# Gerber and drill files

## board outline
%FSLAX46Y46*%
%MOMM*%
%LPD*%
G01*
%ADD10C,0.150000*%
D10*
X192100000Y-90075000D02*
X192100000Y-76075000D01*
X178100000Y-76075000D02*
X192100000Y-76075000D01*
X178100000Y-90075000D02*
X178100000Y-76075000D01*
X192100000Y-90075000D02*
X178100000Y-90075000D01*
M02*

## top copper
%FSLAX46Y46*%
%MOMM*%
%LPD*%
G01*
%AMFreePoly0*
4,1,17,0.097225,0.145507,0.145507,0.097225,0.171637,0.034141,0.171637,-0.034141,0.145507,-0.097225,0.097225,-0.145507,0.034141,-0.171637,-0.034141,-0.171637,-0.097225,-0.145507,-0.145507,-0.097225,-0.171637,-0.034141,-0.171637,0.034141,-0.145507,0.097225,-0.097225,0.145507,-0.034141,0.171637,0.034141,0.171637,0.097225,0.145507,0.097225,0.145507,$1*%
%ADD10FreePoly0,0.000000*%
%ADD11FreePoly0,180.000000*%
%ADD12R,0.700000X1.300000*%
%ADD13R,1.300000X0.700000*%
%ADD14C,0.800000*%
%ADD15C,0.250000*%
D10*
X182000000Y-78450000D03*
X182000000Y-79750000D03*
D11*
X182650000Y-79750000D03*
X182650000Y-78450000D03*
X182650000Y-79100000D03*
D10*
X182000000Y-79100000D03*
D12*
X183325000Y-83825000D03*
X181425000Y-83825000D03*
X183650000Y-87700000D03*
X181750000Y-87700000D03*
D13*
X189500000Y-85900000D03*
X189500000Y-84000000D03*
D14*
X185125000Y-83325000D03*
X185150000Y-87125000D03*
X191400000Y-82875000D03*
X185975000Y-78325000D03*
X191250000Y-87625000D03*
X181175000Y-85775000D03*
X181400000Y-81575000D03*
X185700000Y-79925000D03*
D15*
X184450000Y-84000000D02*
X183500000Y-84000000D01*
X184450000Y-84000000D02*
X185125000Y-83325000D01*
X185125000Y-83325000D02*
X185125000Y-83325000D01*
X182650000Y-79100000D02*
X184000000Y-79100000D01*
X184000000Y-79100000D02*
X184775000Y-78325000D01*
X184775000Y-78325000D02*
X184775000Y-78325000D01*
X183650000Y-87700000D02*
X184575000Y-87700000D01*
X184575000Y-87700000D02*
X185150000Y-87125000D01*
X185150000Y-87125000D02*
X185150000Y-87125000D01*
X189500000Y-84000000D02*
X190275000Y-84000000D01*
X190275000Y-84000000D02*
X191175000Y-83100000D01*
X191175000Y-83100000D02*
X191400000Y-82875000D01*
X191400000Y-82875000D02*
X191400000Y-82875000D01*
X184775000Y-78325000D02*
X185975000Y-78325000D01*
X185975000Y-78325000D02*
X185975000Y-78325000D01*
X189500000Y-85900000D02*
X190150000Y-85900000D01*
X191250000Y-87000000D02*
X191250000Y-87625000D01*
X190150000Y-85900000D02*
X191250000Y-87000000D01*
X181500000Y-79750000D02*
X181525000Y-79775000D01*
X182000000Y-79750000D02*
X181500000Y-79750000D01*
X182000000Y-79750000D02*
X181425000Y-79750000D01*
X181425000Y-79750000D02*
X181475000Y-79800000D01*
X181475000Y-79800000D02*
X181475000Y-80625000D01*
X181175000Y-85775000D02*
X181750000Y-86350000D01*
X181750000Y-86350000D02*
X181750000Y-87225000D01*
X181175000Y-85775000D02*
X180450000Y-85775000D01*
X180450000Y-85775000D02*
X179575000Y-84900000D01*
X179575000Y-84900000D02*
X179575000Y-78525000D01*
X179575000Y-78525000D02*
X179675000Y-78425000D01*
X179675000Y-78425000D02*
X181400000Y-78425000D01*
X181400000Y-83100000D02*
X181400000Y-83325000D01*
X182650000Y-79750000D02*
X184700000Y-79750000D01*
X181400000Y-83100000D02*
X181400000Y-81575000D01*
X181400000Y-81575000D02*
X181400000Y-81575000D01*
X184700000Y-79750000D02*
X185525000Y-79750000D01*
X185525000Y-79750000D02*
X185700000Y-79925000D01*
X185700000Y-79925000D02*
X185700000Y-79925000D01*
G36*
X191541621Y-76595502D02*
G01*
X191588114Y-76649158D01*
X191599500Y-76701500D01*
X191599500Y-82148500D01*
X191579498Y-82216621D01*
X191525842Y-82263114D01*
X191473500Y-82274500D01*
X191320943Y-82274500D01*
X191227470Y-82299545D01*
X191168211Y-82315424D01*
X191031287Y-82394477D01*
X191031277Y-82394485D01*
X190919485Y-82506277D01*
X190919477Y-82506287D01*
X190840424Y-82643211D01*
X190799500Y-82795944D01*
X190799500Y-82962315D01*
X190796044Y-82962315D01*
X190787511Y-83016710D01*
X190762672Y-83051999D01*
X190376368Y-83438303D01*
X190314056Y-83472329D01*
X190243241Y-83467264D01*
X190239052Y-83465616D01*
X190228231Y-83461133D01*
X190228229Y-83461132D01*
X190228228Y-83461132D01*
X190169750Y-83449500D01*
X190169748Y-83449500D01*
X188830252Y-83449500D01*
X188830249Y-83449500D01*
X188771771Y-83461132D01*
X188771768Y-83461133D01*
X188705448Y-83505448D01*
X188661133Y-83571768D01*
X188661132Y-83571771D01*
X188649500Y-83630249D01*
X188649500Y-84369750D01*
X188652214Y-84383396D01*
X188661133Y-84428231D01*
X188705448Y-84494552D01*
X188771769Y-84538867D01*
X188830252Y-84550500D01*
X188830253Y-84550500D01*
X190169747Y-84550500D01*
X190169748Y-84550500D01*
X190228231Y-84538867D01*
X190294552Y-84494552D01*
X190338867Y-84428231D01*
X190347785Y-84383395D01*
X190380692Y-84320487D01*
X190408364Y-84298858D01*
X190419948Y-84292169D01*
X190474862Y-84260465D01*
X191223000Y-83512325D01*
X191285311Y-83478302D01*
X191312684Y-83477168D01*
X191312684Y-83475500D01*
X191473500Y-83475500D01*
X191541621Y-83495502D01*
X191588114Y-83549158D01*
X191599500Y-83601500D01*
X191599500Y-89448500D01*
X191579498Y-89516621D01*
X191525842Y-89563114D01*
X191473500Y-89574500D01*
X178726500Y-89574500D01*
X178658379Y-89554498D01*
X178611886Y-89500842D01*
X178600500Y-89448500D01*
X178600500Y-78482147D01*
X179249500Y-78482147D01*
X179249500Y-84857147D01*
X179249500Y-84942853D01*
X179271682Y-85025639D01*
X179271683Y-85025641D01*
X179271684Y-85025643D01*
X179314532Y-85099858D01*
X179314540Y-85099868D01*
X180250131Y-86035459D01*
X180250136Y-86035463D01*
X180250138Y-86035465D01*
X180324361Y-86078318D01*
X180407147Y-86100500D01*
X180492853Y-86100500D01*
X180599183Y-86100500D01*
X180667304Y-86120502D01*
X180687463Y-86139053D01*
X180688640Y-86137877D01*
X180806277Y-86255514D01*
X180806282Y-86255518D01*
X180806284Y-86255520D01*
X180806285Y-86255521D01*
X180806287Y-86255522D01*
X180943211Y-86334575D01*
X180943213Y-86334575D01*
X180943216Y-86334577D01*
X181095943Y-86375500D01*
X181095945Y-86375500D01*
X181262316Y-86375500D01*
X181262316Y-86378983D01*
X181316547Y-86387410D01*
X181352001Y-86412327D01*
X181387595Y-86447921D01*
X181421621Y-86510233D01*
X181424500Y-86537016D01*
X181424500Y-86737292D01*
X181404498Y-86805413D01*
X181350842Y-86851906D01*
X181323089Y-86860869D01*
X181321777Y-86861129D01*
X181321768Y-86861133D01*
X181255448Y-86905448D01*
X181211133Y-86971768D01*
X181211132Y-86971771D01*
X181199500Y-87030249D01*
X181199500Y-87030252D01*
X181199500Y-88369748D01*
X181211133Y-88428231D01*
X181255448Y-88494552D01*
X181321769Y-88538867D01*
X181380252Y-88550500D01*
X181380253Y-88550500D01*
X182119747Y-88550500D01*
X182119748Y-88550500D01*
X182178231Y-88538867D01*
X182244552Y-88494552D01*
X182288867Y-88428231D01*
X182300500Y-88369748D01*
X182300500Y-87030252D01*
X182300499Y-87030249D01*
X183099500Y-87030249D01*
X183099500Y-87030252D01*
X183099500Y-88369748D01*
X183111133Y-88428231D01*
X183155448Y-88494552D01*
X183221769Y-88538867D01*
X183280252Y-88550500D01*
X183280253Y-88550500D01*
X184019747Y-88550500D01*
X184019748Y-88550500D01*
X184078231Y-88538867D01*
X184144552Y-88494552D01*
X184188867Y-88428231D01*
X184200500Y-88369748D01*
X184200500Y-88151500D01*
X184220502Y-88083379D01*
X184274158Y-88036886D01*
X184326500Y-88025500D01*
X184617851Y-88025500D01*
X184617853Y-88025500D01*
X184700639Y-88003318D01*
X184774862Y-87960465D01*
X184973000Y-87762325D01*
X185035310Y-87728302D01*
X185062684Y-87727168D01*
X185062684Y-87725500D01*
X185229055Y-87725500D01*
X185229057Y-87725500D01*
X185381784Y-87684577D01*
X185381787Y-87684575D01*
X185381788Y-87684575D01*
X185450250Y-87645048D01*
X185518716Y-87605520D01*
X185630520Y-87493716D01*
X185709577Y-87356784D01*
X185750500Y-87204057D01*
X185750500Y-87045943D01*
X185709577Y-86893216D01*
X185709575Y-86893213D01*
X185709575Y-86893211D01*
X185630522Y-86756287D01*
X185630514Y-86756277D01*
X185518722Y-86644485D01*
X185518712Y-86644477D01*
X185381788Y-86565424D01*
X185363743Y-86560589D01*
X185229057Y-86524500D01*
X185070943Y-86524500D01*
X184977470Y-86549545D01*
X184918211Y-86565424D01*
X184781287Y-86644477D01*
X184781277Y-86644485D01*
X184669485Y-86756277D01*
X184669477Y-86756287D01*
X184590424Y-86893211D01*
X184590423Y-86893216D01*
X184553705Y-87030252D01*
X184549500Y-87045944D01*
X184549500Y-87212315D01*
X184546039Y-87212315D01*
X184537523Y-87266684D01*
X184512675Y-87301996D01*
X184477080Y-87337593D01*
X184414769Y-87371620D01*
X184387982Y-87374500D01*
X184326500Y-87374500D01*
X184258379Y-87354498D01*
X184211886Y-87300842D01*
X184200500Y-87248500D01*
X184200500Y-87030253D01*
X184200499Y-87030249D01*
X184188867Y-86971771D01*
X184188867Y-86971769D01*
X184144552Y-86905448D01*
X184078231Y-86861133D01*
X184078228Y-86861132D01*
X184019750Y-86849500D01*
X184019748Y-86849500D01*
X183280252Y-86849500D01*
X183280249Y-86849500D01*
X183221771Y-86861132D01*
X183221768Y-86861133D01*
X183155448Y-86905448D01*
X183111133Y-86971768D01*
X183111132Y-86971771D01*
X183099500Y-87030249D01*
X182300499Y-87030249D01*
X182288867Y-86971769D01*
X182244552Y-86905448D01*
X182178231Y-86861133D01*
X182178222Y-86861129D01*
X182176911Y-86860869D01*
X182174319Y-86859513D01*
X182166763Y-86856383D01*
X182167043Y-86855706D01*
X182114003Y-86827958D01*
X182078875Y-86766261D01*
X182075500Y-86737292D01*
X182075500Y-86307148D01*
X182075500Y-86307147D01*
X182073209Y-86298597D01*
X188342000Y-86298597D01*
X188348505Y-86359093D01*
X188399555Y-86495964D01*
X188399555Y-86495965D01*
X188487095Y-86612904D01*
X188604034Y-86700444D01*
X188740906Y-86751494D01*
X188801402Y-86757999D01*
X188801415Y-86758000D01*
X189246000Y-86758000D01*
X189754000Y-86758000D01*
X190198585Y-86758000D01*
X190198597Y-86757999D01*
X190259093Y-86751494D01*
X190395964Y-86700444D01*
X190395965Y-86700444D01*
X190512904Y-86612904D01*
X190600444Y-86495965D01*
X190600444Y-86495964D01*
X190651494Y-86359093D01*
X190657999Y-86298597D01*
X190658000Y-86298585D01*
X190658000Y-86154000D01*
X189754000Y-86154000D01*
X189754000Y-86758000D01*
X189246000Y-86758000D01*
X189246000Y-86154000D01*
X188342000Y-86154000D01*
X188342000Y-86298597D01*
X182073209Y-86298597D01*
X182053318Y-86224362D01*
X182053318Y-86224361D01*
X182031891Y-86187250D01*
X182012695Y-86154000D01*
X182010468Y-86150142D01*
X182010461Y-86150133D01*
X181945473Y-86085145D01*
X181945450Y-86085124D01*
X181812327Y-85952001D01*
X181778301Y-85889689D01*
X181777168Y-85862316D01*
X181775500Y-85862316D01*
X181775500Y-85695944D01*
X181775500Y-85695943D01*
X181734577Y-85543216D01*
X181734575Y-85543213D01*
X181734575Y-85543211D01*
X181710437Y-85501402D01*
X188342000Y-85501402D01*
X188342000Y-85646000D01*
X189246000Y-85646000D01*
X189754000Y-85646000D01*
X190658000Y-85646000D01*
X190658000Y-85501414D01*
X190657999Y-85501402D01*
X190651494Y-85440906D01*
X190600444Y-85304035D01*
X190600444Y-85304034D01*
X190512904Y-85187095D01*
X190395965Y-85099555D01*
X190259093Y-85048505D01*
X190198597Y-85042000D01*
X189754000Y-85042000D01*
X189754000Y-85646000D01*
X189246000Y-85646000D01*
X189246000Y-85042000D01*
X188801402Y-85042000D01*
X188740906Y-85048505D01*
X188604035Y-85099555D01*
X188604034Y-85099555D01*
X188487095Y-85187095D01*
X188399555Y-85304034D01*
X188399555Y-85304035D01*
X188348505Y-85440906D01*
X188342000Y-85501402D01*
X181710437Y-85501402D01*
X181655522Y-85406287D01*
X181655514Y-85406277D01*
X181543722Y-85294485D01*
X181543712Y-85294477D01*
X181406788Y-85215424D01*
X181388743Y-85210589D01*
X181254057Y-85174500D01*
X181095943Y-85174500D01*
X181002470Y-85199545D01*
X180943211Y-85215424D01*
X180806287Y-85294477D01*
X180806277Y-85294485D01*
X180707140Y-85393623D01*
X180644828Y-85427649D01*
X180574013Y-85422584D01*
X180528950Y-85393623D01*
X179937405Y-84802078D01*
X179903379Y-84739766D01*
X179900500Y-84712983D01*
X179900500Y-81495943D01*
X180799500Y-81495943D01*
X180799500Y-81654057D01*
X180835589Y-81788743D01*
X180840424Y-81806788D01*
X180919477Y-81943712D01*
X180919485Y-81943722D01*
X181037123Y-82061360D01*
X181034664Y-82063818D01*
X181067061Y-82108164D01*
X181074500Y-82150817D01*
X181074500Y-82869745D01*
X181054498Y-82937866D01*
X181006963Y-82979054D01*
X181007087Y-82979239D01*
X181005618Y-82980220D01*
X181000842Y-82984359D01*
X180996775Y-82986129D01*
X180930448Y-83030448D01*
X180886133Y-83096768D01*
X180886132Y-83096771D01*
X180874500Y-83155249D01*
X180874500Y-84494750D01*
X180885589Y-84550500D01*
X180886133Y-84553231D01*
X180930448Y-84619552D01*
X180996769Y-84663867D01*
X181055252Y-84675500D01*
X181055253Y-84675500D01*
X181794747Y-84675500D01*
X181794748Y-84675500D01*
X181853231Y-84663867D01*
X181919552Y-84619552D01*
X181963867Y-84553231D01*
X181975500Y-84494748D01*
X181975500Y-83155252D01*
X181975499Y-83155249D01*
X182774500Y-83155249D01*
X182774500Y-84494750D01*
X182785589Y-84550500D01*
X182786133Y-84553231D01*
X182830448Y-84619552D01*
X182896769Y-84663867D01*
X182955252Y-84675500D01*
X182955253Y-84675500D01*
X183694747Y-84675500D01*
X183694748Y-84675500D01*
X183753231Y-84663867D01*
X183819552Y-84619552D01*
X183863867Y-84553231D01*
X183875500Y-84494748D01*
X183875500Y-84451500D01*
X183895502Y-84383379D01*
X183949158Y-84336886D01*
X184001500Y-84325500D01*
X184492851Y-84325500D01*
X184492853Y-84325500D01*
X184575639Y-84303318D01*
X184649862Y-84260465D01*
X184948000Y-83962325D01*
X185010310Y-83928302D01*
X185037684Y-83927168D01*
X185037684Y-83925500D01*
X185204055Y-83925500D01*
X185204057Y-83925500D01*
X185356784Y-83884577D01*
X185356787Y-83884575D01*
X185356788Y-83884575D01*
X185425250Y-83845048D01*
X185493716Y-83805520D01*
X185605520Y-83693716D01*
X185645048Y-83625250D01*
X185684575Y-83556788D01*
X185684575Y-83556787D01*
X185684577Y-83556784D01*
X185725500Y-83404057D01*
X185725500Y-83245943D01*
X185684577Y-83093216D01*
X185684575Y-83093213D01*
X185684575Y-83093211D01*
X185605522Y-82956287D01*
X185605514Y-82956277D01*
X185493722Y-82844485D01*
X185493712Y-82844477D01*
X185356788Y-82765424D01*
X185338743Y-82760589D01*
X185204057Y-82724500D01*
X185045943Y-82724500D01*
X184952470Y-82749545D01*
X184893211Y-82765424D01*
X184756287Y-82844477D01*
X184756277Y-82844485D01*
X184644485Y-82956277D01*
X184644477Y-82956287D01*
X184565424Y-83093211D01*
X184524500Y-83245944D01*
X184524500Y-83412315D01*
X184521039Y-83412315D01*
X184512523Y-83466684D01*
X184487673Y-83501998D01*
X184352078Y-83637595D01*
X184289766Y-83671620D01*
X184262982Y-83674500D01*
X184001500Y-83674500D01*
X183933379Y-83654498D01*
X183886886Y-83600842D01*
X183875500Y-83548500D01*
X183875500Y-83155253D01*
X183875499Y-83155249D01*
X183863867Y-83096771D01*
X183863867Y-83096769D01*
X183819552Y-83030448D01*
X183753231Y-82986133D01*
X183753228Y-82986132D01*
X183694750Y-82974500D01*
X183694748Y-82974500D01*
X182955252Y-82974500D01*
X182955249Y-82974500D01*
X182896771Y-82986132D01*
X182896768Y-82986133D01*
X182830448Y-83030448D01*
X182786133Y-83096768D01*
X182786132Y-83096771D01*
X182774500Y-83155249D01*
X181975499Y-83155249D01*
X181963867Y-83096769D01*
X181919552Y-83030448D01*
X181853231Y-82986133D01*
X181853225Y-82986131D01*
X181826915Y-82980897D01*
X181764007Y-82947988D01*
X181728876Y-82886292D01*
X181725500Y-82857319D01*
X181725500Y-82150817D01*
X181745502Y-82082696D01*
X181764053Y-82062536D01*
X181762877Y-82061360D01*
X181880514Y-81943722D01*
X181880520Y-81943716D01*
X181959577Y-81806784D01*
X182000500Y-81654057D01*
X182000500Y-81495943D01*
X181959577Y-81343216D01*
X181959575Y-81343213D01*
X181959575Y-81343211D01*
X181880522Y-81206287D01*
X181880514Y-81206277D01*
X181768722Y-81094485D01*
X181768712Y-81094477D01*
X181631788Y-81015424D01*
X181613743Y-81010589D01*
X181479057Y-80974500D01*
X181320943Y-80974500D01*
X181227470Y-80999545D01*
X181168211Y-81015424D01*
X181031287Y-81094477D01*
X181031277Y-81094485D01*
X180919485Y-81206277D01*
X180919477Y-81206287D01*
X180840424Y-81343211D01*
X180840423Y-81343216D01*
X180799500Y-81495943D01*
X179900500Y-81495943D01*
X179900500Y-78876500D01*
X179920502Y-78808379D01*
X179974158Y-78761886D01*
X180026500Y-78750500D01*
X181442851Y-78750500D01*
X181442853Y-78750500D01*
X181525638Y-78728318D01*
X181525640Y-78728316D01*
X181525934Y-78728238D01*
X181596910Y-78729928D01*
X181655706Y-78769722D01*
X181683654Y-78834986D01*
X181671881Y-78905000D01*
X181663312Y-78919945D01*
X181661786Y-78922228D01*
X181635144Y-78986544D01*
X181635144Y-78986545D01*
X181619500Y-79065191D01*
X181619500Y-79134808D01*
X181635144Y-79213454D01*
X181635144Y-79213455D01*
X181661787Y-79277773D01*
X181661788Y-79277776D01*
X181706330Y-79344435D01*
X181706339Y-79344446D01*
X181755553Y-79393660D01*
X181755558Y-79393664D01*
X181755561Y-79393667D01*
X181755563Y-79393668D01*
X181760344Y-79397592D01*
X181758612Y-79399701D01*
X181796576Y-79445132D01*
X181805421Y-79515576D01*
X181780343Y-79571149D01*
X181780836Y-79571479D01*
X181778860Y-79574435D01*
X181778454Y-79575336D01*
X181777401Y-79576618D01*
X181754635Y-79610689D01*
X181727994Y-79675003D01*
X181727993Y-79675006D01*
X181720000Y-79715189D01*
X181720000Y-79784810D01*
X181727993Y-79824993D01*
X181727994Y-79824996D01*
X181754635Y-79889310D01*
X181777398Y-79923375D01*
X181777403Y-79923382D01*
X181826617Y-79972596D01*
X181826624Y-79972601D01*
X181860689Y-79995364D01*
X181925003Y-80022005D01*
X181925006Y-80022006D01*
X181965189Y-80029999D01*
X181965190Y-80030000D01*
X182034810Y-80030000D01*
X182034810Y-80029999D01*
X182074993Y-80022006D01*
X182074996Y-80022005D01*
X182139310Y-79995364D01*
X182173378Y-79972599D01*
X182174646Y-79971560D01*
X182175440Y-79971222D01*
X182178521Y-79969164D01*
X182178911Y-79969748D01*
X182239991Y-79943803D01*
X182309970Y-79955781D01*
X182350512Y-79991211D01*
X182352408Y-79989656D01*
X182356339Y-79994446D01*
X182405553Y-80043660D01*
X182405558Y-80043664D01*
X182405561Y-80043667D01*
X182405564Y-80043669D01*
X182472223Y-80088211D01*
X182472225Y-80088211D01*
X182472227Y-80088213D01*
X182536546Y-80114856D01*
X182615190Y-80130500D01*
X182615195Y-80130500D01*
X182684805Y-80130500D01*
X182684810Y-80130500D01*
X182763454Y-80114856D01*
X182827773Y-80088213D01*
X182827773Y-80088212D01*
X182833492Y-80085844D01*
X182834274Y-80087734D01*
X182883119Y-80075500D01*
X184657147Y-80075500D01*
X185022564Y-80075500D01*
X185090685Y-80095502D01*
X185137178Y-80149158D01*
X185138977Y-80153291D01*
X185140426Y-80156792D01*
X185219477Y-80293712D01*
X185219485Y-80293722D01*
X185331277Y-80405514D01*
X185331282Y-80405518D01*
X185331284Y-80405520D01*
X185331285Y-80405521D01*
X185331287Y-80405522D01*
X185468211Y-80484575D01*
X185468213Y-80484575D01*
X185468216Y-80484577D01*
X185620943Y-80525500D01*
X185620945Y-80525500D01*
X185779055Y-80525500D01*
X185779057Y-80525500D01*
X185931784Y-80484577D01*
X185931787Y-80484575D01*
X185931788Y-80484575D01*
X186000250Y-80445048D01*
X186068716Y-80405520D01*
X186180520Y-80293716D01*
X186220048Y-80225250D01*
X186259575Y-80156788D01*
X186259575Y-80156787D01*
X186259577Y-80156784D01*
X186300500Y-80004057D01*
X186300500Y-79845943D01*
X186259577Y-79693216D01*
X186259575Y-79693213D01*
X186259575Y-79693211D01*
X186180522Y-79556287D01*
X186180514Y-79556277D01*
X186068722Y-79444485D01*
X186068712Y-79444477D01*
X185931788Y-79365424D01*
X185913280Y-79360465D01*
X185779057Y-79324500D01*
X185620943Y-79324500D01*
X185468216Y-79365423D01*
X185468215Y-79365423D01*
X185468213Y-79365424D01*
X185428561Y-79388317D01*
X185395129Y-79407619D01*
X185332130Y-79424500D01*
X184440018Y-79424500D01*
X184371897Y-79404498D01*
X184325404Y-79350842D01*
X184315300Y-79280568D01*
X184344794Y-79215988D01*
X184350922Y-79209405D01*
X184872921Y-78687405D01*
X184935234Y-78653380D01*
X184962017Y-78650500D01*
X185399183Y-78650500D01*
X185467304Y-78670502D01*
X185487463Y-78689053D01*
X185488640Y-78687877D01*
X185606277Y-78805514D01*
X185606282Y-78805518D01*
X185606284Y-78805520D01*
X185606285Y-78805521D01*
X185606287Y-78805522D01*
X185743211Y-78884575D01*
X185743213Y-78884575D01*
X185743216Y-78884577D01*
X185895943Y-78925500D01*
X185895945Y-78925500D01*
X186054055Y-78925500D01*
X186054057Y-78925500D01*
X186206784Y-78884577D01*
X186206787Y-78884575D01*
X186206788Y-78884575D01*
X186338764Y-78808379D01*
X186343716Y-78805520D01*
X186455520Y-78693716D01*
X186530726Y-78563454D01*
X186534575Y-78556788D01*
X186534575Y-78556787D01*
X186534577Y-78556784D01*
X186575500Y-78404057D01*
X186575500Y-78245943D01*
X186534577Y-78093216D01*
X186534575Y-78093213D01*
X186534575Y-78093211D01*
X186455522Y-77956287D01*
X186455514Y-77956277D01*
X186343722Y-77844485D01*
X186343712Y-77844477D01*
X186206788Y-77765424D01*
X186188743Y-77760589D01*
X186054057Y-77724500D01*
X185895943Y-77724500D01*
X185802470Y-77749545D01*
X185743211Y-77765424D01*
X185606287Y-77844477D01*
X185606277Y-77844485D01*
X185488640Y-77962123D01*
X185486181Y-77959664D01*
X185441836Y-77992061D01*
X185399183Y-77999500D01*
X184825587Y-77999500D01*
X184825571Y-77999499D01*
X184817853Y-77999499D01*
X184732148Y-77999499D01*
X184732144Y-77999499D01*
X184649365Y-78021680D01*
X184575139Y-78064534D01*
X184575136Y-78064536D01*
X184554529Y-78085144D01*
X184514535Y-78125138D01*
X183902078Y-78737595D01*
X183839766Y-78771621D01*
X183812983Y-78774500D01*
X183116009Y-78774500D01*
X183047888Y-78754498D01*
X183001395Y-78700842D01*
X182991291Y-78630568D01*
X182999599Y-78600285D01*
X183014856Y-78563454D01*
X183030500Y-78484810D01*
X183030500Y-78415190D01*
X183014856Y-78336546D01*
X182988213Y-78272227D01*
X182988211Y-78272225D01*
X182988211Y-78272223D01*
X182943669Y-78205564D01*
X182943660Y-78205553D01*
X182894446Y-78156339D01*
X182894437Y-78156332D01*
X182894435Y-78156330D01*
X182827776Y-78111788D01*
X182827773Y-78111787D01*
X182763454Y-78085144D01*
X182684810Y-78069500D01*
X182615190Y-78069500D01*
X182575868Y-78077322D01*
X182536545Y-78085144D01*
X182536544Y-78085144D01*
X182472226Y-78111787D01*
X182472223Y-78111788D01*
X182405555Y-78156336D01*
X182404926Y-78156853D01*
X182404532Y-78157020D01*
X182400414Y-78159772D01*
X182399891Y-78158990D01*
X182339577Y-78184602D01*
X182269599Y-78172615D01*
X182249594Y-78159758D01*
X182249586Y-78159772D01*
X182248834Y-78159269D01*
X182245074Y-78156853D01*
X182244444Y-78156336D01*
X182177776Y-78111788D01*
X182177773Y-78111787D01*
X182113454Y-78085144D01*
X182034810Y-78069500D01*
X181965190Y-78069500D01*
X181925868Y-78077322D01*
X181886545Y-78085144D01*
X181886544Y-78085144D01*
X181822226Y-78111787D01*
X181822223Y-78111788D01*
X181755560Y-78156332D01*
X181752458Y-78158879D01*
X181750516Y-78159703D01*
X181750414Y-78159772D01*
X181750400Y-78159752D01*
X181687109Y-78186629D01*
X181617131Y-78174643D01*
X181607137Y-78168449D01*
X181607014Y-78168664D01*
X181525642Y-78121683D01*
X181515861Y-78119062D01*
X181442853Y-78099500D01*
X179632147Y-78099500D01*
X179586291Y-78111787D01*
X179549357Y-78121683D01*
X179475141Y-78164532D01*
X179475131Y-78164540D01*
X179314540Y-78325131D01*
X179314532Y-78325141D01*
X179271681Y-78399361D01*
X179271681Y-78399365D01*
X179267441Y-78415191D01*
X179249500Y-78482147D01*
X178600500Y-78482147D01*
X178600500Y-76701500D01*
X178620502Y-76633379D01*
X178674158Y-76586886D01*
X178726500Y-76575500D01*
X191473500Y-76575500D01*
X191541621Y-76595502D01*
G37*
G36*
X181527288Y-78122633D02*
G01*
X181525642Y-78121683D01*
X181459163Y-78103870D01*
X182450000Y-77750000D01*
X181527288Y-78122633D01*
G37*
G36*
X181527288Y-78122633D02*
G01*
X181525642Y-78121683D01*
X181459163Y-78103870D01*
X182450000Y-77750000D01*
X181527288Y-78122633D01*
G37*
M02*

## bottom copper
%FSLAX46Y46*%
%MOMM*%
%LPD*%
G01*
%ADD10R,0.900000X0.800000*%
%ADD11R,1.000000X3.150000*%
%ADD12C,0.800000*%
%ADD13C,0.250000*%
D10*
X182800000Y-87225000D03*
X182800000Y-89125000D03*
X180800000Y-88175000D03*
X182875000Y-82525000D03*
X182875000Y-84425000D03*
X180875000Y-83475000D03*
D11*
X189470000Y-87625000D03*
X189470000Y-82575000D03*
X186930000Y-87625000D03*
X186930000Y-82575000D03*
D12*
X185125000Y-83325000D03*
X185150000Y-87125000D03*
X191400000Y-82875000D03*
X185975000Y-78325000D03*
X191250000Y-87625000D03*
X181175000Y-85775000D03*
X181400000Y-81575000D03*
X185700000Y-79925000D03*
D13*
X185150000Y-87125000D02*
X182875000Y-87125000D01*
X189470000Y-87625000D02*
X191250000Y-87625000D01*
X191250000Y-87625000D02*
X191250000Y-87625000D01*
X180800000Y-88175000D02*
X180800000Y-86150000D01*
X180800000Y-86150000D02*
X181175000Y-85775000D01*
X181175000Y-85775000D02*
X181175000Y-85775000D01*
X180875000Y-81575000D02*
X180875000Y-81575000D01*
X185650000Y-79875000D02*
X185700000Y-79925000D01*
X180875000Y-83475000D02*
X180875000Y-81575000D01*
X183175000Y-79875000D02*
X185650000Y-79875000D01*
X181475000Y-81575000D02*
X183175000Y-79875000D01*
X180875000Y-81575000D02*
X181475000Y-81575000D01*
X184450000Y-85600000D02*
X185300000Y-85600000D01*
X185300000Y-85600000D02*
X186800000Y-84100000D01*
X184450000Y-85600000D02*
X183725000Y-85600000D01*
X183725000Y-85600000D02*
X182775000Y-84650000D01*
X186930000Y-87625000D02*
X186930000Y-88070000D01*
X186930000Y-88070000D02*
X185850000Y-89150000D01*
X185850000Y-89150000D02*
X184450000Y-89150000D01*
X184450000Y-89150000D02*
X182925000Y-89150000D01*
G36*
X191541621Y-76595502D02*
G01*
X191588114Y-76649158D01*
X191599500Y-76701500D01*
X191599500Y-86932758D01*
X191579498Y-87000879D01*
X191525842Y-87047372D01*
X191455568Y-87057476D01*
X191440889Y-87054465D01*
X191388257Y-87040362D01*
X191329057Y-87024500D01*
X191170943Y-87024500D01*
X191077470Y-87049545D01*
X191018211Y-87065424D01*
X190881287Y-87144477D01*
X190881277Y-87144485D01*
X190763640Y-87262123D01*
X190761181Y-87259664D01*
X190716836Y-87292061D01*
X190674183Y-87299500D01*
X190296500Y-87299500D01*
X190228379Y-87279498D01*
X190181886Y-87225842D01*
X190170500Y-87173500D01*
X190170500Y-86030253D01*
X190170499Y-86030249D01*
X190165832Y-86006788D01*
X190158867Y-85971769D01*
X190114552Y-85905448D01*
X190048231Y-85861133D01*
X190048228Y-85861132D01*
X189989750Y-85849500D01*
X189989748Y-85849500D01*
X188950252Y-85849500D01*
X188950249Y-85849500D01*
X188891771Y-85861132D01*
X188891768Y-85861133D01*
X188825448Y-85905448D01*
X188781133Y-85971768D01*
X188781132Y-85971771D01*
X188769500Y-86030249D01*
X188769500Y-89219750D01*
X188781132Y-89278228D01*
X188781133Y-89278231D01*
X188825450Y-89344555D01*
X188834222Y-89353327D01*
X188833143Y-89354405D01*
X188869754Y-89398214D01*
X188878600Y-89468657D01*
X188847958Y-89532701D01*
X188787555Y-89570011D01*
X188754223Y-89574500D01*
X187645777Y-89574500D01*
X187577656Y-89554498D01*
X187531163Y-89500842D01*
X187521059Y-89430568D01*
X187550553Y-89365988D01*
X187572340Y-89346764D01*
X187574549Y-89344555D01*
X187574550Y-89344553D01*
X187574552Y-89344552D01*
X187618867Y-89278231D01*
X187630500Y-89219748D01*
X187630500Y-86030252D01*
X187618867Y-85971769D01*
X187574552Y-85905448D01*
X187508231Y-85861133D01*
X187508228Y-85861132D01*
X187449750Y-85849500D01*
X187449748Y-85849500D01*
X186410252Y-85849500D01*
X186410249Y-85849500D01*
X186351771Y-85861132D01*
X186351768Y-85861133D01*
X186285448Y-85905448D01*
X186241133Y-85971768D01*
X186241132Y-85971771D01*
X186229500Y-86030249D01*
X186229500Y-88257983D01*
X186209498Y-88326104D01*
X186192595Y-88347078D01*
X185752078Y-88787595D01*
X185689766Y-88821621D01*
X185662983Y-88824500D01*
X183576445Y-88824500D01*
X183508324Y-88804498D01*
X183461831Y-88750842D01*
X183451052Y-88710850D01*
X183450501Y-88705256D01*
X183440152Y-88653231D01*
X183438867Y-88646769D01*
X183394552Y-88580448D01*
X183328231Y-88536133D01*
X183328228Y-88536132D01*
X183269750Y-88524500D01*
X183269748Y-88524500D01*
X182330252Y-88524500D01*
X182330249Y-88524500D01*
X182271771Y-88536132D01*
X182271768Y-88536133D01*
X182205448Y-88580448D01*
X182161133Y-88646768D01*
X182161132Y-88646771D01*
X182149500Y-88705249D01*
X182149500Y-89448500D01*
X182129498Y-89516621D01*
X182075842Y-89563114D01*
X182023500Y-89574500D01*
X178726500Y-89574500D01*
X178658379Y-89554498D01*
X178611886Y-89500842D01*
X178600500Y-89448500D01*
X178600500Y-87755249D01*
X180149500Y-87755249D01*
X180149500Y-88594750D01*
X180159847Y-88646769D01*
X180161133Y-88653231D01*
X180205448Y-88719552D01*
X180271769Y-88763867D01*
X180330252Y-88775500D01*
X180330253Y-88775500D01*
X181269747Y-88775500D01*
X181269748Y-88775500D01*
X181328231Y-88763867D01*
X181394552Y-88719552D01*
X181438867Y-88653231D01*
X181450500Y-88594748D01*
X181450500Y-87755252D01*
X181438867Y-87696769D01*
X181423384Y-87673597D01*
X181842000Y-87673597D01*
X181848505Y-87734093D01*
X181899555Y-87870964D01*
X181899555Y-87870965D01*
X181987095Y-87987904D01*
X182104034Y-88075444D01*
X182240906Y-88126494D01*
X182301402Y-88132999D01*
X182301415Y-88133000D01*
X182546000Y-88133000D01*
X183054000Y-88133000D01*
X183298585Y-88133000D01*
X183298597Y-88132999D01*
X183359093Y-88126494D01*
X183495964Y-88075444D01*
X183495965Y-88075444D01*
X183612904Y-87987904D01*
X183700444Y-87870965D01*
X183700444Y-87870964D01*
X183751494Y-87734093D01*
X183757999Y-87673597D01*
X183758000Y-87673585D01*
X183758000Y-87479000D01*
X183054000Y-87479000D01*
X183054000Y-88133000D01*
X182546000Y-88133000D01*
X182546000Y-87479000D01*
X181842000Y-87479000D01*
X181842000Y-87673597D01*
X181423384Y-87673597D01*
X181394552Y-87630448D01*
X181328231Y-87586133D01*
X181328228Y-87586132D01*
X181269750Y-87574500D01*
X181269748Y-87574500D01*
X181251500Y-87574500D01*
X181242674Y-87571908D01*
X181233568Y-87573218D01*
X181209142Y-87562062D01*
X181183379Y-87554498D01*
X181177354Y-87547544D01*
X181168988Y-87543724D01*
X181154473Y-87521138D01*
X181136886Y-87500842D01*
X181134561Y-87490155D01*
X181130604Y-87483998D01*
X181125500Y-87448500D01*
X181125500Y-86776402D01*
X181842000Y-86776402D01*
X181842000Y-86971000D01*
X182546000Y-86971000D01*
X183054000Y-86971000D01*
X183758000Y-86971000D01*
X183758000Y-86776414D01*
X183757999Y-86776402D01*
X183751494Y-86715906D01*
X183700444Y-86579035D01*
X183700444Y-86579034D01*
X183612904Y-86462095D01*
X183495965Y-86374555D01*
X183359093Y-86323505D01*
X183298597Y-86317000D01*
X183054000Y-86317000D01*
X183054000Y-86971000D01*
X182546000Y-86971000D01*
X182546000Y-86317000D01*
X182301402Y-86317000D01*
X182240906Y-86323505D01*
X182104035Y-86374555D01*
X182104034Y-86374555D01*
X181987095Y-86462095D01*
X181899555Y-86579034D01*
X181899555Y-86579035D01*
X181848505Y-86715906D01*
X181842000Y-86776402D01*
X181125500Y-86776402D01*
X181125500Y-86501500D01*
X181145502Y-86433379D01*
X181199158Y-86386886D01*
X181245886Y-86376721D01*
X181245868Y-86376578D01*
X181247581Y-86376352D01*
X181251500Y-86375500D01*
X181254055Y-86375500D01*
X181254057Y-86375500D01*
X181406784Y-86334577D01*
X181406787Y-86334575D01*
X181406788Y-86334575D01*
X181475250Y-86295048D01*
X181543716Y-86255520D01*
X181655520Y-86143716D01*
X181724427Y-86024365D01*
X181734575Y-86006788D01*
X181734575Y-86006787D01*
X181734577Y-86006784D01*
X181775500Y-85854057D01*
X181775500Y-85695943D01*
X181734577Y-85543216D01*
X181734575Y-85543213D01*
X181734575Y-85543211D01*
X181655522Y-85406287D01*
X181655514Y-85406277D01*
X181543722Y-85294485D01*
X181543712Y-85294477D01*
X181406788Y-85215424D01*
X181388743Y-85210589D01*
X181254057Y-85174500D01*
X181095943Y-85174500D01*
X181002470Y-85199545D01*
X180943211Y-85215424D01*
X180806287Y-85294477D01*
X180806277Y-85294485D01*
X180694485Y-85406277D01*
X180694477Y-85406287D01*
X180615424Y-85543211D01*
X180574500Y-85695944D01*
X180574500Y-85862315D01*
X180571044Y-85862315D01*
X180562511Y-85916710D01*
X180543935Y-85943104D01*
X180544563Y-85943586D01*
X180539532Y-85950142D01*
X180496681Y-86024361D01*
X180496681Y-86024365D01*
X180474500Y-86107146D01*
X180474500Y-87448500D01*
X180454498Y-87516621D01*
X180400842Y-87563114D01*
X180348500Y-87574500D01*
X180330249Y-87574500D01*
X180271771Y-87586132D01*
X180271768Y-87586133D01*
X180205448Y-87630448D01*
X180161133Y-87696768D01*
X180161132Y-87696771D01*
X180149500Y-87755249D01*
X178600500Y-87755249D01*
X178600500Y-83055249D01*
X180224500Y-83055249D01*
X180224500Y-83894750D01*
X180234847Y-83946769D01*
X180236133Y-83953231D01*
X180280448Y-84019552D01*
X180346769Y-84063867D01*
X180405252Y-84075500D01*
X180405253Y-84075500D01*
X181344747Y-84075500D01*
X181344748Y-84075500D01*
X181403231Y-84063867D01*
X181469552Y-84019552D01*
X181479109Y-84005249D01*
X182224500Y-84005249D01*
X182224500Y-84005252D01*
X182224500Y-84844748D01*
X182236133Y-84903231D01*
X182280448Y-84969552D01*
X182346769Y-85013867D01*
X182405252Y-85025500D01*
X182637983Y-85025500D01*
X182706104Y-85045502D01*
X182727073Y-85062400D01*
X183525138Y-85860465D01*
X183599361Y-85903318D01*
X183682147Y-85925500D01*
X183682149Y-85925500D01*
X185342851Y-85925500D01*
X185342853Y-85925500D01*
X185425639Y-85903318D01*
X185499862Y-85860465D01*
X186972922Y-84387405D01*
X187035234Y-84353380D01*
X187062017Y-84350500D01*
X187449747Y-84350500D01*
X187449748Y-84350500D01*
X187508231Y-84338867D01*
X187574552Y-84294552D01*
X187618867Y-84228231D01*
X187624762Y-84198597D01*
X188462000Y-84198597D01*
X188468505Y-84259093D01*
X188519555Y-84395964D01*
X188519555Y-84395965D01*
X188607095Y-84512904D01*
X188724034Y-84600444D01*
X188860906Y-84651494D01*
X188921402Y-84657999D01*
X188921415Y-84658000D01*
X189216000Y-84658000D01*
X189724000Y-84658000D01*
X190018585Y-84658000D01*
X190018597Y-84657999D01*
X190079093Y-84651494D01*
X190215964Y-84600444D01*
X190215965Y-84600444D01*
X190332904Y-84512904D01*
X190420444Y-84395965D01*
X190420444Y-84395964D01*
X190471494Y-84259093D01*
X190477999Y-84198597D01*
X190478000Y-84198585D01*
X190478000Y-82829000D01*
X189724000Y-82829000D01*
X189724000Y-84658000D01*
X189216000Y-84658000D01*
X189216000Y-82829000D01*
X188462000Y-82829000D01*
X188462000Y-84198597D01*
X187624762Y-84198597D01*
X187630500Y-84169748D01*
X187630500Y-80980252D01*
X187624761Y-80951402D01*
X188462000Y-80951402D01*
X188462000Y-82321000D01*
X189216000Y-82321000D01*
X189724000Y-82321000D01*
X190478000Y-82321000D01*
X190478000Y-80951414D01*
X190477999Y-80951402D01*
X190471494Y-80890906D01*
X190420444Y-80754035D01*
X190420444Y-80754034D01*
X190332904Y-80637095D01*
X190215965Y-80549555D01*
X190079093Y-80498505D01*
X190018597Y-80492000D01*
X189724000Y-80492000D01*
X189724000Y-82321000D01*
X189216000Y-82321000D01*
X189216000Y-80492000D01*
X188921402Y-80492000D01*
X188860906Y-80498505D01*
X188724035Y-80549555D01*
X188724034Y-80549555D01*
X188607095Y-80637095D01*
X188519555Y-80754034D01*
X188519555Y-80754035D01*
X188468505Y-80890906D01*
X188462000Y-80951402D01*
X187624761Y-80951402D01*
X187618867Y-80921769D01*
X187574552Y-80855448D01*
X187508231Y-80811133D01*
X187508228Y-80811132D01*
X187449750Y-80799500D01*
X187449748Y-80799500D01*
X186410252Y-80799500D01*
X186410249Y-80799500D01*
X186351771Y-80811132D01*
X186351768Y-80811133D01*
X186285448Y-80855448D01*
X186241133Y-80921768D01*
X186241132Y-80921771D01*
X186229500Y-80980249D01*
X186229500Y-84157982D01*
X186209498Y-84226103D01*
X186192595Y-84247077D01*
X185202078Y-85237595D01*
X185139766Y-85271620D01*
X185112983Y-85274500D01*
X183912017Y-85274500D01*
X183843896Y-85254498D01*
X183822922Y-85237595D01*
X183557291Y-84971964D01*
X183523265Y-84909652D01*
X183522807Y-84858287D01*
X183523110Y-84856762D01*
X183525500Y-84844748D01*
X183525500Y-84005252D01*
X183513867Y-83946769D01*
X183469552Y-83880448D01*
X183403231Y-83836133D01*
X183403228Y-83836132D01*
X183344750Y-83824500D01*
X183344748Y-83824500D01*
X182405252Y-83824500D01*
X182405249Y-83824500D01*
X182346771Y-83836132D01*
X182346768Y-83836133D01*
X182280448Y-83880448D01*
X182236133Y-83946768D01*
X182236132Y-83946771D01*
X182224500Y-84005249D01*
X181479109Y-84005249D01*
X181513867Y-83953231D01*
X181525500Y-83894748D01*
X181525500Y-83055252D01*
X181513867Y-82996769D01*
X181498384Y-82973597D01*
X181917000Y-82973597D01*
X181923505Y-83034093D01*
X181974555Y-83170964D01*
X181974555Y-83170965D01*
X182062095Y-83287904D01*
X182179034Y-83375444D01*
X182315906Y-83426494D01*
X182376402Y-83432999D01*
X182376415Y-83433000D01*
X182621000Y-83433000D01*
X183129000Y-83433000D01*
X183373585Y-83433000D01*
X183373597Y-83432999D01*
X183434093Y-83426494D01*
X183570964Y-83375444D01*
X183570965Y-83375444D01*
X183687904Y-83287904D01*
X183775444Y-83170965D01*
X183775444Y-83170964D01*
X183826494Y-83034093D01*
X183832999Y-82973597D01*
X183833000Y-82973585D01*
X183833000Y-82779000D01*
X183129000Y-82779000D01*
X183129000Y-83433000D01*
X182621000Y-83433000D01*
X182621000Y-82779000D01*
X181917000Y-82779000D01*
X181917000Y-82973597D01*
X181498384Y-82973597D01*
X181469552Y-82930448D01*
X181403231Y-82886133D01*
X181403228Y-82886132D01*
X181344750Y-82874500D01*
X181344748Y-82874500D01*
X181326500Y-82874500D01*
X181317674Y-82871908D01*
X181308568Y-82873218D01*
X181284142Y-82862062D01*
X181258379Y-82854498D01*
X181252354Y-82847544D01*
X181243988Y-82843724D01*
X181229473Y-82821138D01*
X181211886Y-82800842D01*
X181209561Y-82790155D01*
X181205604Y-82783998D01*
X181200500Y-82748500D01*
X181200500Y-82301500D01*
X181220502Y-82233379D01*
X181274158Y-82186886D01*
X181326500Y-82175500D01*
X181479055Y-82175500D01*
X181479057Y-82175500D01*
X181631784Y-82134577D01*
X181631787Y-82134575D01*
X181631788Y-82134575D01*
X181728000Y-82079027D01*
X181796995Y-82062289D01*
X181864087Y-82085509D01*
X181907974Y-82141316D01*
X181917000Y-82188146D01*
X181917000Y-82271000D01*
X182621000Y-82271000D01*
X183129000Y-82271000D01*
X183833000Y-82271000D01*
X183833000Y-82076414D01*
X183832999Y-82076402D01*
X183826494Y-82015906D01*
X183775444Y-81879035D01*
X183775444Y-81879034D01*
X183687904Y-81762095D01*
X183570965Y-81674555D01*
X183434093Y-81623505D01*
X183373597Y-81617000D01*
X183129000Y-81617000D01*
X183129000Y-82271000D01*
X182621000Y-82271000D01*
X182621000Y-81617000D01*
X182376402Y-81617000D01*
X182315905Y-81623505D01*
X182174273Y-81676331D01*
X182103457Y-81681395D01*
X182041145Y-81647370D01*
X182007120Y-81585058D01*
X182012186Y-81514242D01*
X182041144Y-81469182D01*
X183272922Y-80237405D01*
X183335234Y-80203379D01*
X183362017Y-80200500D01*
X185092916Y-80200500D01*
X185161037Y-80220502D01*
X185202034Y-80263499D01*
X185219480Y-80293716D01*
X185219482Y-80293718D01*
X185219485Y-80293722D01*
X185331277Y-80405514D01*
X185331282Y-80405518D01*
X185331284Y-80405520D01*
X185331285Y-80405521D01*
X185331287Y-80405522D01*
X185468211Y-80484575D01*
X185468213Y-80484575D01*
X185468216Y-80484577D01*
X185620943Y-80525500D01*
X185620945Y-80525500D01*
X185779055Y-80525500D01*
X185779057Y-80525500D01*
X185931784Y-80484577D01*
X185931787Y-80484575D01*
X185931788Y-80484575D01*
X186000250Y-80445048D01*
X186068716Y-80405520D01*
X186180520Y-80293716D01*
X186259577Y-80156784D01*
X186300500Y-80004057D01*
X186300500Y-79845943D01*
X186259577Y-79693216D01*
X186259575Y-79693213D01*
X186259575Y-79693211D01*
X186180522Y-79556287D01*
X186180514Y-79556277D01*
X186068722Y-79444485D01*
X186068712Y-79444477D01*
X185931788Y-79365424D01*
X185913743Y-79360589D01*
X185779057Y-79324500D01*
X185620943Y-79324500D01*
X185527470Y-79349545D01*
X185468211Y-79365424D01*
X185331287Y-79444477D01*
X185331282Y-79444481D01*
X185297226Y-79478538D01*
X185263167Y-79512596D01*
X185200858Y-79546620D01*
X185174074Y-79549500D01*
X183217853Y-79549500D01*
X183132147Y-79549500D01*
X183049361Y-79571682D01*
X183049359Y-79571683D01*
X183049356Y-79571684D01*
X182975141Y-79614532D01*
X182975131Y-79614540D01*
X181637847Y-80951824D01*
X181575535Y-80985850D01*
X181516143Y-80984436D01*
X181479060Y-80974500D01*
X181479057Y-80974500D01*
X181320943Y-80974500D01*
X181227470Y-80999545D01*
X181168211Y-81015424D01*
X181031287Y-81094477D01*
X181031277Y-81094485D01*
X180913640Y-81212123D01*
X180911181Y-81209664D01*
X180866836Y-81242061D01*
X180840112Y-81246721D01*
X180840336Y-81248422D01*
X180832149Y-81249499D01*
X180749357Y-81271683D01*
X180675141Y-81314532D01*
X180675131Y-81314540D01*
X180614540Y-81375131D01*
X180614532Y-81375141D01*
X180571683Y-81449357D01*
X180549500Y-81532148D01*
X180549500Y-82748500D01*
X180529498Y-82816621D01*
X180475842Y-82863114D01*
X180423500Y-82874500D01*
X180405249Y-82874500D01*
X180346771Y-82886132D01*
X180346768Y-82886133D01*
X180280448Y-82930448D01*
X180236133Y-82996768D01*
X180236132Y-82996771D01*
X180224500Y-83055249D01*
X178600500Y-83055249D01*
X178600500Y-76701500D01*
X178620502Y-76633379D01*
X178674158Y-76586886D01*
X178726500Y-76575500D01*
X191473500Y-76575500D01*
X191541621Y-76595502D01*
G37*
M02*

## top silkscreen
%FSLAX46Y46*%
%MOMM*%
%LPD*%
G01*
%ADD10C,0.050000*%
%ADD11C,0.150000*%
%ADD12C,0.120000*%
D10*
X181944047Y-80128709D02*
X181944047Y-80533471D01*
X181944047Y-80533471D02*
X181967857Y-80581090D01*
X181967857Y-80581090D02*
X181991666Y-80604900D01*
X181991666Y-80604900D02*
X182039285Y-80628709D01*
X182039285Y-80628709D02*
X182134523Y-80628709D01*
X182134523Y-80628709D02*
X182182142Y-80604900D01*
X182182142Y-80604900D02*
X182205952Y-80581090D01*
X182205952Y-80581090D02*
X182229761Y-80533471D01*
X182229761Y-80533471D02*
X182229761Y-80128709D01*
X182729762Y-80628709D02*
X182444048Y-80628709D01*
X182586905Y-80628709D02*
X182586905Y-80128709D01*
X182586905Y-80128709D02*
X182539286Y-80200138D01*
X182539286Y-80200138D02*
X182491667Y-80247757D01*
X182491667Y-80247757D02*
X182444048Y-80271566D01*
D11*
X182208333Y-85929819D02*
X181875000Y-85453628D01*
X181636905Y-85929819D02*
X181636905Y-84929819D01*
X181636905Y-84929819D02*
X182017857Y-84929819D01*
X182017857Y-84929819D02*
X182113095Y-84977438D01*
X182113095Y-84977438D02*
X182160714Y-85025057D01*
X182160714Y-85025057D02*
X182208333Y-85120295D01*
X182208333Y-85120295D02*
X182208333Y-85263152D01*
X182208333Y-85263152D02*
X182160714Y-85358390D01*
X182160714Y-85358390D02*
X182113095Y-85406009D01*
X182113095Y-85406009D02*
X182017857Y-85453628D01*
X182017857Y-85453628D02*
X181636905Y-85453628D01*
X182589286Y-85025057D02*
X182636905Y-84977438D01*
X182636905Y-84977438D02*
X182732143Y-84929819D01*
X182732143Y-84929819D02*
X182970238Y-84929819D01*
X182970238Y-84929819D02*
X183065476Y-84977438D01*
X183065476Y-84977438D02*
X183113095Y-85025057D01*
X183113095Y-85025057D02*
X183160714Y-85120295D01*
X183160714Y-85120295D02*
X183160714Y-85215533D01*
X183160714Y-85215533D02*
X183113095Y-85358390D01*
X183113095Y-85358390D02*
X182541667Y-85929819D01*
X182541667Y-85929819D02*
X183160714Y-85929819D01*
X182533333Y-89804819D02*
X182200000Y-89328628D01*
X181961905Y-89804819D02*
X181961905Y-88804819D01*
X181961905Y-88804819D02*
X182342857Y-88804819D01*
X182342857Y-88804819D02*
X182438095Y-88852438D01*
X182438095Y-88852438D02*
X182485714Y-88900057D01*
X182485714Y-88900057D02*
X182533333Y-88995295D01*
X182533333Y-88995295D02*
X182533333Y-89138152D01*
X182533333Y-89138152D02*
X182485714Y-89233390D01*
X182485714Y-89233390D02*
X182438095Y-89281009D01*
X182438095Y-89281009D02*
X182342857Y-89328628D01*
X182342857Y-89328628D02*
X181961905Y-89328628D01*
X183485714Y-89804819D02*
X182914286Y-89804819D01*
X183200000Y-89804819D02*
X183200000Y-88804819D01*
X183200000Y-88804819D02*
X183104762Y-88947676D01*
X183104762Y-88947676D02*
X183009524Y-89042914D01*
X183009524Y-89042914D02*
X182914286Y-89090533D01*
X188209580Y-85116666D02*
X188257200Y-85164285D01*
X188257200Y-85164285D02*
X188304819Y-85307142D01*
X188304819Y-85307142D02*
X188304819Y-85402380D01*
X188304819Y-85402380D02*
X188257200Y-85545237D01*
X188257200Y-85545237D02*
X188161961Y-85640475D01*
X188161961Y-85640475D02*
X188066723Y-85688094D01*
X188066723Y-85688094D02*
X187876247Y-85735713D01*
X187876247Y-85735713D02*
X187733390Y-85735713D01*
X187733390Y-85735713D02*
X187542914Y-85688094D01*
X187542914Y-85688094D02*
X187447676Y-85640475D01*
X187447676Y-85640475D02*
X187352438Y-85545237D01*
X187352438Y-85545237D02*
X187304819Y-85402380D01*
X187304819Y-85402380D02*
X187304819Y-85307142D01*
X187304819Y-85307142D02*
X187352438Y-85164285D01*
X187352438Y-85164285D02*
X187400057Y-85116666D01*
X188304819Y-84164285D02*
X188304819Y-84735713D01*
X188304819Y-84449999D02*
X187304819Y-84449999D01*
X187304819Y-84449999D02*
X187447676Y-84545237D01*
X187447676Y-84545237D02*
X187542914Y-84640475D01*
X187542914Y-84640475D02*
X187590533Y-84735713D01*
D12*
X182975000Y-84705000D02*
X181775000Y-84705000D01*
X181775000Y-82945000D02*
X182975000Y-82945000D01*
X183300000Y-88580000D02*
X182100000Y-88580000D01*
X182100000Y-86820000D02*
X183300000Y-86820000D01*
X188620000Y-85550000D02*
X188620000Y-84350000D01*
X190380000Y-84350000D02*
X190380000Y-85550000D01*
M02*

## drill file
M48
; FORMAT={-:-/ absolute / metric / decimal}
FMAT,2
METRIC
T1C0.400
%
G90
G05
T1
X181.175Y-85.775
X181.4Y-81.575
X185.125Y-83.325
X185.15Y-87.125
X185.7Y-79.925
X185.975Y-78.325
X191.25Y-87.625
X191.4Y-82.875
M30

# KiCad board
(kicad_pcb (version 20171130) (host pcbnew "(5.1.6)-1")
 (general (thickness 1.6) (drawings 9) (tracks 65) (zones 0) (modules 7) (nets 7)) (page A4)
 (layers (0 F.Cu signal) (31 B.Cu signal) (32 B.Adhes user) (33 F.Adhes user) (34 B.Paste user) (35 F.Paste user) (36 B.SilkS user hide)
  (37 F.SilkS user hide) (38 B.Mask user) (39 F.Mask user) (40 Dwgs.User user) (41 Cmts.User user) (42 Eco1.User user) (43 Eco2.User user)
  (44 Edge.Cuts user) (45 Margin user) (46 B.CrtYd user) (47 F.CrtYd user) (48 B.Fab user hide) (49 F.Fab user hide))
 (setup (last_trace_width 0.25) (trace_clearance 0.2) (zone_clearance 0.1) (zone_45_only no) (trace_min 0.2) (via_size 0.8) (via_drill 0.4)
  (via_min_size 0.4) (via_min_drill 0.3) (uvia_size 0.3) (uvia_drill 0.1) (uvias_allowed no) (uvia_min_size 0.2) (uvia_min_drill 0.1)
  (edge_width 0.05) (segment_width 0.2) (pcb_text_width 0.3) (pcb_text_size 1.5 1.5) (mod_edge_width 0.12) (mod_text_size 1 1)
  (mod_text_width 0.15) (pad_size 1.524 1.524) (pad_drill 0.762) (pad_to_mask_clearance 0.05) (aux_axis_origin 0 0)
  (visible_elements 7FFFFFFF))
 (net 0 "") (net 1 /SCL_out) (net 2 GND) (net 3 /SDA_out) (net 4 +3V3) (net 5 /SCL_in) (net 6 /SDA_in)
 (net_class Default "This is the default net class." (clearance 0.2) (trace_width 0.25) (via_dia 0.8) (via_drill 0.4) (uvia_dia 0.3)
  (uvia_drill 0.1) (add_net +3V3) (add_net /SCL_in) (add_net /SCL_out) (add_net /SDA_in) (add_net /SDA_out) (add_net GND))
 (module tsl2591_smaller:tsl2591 (layer F.Cu) (at 182.325 79.1)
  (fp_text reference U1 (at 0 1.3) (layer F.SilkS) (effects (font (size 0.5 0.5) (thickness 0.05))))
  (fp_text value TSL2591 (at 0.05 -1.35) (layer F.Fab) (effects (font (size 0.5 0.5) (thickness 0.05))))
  (pad 1 smd custom (at -0.325 -0.65) (size 0.35 0.35) (layers F.Cu F.Paste F.Mask) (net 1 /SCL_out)
   (options (clearance outline) (anchor circle)) (primitives))
  (pad 3 smd custom (at -0.325 0.65) (size 0.35 0.35) (layers F.Cu F.Paste F.Mask) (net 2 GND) (zone_connect 0)
   (options (clearance outline) (anchor circle)) (primitives))
  (pad 6 smd custom (at 0.325 0.65 180) (size 0.35 0.35) (layers F.Cu F.Paste F.Mask) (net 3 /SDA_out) (zone_connect 0)
   (options (clearance outline) (anchor circle)) (primitives))
  (pad 4 smd custom (at 0.325 -0.65 180) (size 0.35 0.35) (layers F.Cu F.Paste F.Mask) (zone_connect 0)
   (options (clearance outline) (anchor circle)) (primitives))
  (pad 5 smd custom (at 0.325 0 180) (size 0.35 0.35) (layers F.Cu F.Paste F.Mask) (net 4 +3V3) (zone_connect 0)
   (options (clearance outline) (anchor circle)) (primitives))
  (pad 2 smd custom (at -0.325 0) (size 0.35 0.35) (layers F.Cu F.Paste F.Mask) (options (clearance outline) (anchor circle)) (primitives)))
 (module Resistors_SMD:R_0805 (layer F.Cu) (at 182.375 83.825 180)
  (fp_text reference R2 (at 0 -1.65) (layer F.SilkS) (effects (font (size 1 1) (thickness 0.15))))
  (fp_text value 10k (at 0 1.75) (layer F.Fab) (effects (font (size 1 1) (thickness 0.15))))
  (fp_line (start -0.6 -0.88) (end 0.6 -0.88) (layer F.SilkS) (width 0.12))
  (fp_line (start 0.6 0.88) (end -0.6 0.88) (layer F.SilkS) (width 0.12))
  (pad 1 smd rect (at -0.95 0 180) (size 0.7 1.3) (layers F.Cu F.Paste F.Mask) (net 4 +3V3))
  (pad 2 smd rect (at 0.95 0 180) (size 0.7 1.3) (layers F.Cu F.Paste F.Mask) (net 3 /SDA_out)))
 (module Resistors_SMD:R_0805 (layer F.Cu) (at 182.7 87.7 180)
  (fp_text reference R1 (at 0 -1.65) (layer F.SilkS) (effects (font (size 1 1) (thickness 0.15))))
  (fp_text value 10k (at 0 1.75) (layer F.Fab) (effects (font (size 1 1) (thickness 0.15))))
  (fp_line (start -0.6 -0.88) (end 0.6 -0.88) (layer F.SilkS) (width 0.12))
  (fp_line (start 0.6 0.88) (end -0.6 0.88) (layer F.SilkS) (width 0.12))
  (pad 1 smd rect (at -0.95 0 180) (size 0.7 1.3) (layers F.Cu F.Paste F.Mask) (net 4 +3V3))
  (pad 2 smd rect (at 0.95 0 180) (size 0.7 1.3) (layers F.Cu F.Paste F.Mask) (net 1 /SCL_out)))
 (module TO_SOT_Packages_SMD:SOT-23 (layer B.Cu) (at 181.8 88.175 180)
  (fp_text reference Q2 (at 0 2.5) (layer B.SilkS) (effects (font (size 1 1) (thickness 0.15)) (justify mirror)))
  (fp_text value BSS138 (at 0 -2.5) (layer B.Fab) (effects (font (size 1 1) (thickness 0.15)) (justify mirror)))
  (pad 1 smd rect (at -1 0.95 180) (size 0.9 0.8) (layers B.Cu B.Paste B.Mask) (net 4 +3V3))
  (pad 2 smd rect (at -1 -0.95 180) (size 0.9 0.8) (layers B.Cu B.Paste B.Mask) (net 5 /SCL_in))
  (pad 3 smd rect (at 1 0 180) (size 0.9 0.8) (layers B.Cu B.Paste B.Mask) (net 1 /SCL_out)))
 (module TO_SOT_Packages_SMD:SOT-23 (layer B.Cu) (at 181.875 83.475 180)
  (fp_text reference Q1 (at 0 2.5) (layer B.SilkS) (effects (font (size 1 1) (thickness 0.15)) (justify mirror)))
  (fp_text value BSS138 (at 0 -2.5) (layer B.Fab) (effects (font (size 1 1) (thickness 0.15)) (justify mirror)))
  (pad 1 smd rect (at -1 0.95 180) (size 0.9 0.8) (layers B.Cu B.Paste B.Mask) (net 4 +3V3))
  (pad 2 smd rect (at -1 -0.95 180) (size 0.9 0.8) (layers B.Cu B.Paste B.Mask) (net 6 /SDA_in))
  (pad 3 smd rect (at 1 0 180) (size 0.9 0.8) (layers B.Cu B.Paste B.Mask) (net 3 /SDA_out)))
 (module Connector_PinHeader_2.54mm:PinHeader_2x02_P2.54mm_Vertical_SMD (layer B.Cu) (at 188.2 85.1 270)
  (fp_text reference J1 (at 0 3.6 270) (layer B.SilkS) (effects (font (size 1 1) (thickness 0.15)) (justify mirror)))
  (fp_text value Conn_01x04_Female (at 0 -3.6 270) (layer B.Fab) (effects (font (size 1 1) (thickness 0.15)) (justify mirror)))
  (pad 4 smd rect (at 2.525 -1.27 270) (size 3.15 1) (layers B.Cu B.Paste B.Mask) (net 2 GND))
  (pad 3 smd rect (at -2.525 -1.27 270) (size 3.15 1) (layers B.Cu B.Paste B.Mask) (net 4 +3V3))
  (pad 2 smd rect (at 2.525 1.27 270) (size 3.15 1) (layers B.Cu B.Paste B.Mask) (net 5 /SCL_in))
  (pad 1 smd rect (at -2.525 1.27 270) (size 3.15 1) (layers B.Cu B.Paste B.Mask) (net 6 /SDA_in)))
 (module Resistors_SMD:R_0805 (layer F.Cu) (at 189.5 84.95 90)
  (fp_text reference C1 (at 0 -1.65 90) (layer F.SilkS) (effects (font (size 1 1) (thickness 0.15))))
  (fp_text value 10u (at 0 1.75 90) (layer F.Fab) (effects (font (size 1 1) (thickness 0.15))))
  (fp_line (start -0.6 -0.88) (end 0.6 -0.88) (layer F.SilkS) (width 0.12))
  (fp_line (start 0.6 0.88) (end -0.6 0.88) (layer F.SilkS) (width 0.12))
  (pad 1 smd rect (at -0.95 0 90) (size 0.7 1.3) (layers F.Cu F.Paste F.Mask) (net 2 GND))
  (pad 2 smd rect (at 0.95 0 90) (size 0.7 1.3) (layers F.Cu F.Paste F.Mask) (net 4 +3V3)))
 (gr_line (start 192.1 90.075) (end 192.1 76.075) (layer Edge.Cuts) (width 0.15))
 (gr_line (start 178.1 76.075) (end 192.1 76.075) (layer Edge.Cuts) (width 0.15))
 (gr_line (start 178.1 90.075) (end 178.1 76.075) (layer Edge.Cuts) (width 0.15))
 (gr_line (start 192.1 90.075) (end 178.1 90.075) (layer Edge.Cuts) (width 0.15))
 (segment (start 184.45 84) (end 183.5 84) (width 0.25) (layer F.Cu) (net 4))
 (segment (start 184.45 84) (end 185.125 83.325) (width 0.25) (layer F.Cu) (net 4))
 (segment (start 185.125 83.325) (end 185.125 83.325) (width 0.25) (layer F.Cu) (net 4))
 (via (at 185.125 83.325) (size 0.8) (drill 0.4) (layers F.Cu B.Cu) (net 4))
 (segment (start 182.65 79.1) (end 184 79.1) (width 0.25) (layer F.Cu) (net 4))
 (segment (start 184 79.1) (end 184.775 78.325) (width 0.25) (layer F.Cu) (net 4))
 (segment (start 184.775 78.325) (end 184.775 78.325) (width 0.25) (layer F.Cu) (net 4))
 (segment (start 183.65 87.7) (end 184.575 87.7) (width 0.25) (layer F.Cu) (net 4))
 (segment (start 184.575 87.7) (end 185.15 87.125) (width 0.25) (layer F.Cu) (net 4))
 (segment (start 185.15 87.125) (end 185.15 87.125) (width 0.25) (layer F.Cu) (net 4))
 (via (at 185.15 87.125) (size 0.8) (drill 0.4) (layers F.Cu B.Cu) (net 4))
 (segment (start 185.15 87.125) (end 182.875 87.125) (width 0.25) (layer B.Cu) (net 4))
 (segment (start 189.5 84) (end 190.275 84) (width 0.25) (layer F.Cu) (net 4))
 (segment (start 190.275 84) (end 191.175 83.1) (width 0.25) (layer F.Cu) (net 4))
 (segment (start 191.175 83.1) (end 191.4 82.875) (width 0.25) (layer F.Cu) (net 4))
 (segment (start 191.4 82.875) (end 191.4 82.875) (width 0.25) (layer F.Cu) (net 4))
 (via (at 191.4 82.875) (size 0.8) (drill 0.4) (layers F.Cu B.Cu) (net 4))
 (segment (start 184.775 78.325) (end 185.975 78.325) (width 0.25) (layer F.Cu) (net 4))
 (segment (start 185.975 78.325) (end 185.975 78.325) (width 0.25) (layer F.Cu) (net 4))
 (via (at 185.975 78.325) (size 0.8) (drill 0.4) (layers F.Cu B.Cu) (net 4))
 (segment (start 189.47 87.625) (end 191.25 87.625) (width 0.25) (layer B.Cu) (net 2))
 (segment (start 191.25 87.625) (end 191.25 87.625) (width 0.25) (layer B.Cu) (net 2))
 (via (at 191.25 87.625) (size 0.8) (drill 0.4) (layers F.Cu B.Cu) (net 2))
 (segment (start 189.5 85.9) (end 190.15 85.9) (width 0.25) (layer F.Cu) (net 2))
 (segment (start 191.25 87) (end 191.25 87.625) (width 0.25) (layer F.Cu) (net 2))
 (segment (start 190.15 85.9) (end 191.25 87) (width 0.25) (layer F.Cu) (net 2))
 (segment (start 181.5 79.75) (end 181.525 79.775) (width 0.25) (layer F.Cu) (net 2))
 (segment (start 182 79.75) (end 181.5 79.75) (width 0.25) (layer F.Cu) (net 2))
 (segment (start 182 79.75) (end 181.425 79.75) (width 0.25) (layer F.Cu) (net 2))
 (segment (start 181.425 79.75) (end 181.475 79.8) (width 0.25) (layer F.Cu) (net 2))
 (segment (start 181.475 79.8) (end 181.475 80.625) (width 0.25) (layer F.Cu) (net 2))
 (segment (start 180.8 88.175) (end 180.8 86.15) (width 0.25) (layer B.Cu) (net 1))
 (segment (start 180.8 86.15) (end 181.175 85.775) (width 0.25) (layer B.Cu) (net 1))
 (segment (start 181.175 85.775) (end 181.175 85.775) (width 0.25) (layer B.Cu) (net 1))
 (via (at 181.175 85.775) (size 0.8) (drill 0.4) (layers F.Cu B.Cu) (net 1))
 (segment (start 181.175 85.775) (end 181.75 86.35) (width 0.25) (layer F.Cu) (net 1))
 (segment (start 181.75 86.35) (end 181.75 87.225) (width 0.25) (layer F.Cu) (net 1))
 (segment (start 181.175 85.775) (end 180.45 85.775) (width 0.25) (layer F.Cu) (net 1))
 (segment (start 180.45 85.775) (end 179.575 84.9) (width 0.25) (layer F.Cu) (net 1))
 (segment (start 179.575 84.9) (end 179.575 78.525) (width 0.25) (layer F.Cu) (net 1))
 (segment (start 179.575 78.525) (end 179.675 78.425) (width 0.25) (layer F.Cu) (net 1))
 (segment (start 179.675 78.425) (end 181.4 78.425) (width 0.25) (layer F.Cu) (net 1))
 (segment (start 180.875 81.575) (end 180.875 81.575) (width 0.25) (layer B.Cu) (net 3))
 (segment (start 181.4 83.1) (end 181.4 83.325) (width 0.25) (layer F.Cu) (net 3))
 (segment (start 182.65 79.75) (end 184.7 79.75) (width 0.25) (layer F.Cu) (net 3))
 (segment (start 181.4 83.1) (end 181.4 81.575) (width 0.25) (layer F.Cu) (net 3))
 (segment (start 181.4 81.575) (end 181.4 81.575) (width 0.25) (layer F.Cu) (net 3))
 (via (at 181.4 81.575) (size 0.8) (drill 0.4) (layers F.Cu B.Cu) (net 3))
 (segment (start 184.7 79.75) (end 185.525 79.75) (width 0.25) (layer F.Cu) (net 3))
 (segment (start 185.525 79.75) (end 185.7 79.925) (width 0.25) (layer F.Cu) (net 3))
 (segment (start 185.7 79.925) (end 185.7 79.925) (width 0.25) (layer F.Cu) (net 3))
 (via (at 185.7 79.925) (size 0.8) (drill 0.4) (layers F.Cu B.Cu) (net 3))
 (segment (start 185.65 79.875) (end 185.7 79.925) (width 0.25) (layer B.Cu) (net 3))
 (segment (start 180.875 83.475) (end 180.875 81.575) (width 0.25) (layer B.Cu) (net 3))
 (segment (start 183.175 79.875) (end 185.65 79.875) (width 0.25) (layer B.Cu) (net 3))
 (segment (start 181.475 81.575) (end 183.175 79.875) (width 0.25) (layer B.Cu) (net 3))
 (segment (start 180.875 81.575) (end 181.475 81.575) (width 0.25) (layer B.Cu) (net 3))
 (segment (start 184.45 85.6) (end 185.3 85.6) (width 0.25) (layer B.Cu) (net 6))
 (segment (start 185.3 85.6) (end 186.8 84.1) (width 0.25) (layer B.Cu) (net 6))
 (segment (start 184.45 85.6) (end 183.725 85.6) (width 0.25) (layer B.Cu) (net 6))
 (segment (start 183.725 85.6) (end 182.775 84.65) (width 0.25) (layer B.Cu) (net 6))
 (segment (start 186.93 87.625) (end 186.93 88.07) (width 0.25) (layer B.Cu) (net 5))
 (segment (start 186.93 88.07) (end 185.85 89.15) (width 0.25) (layer B.Cu) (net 5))
 (segment (start 185.85 89.15) (end 184.45 89.15) (width 0.25) (layer B.Cu) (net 5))
 (segment (start 184.45 89.15) (end 182.925 89.15) (width 0.25) (layer B.Cu) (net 5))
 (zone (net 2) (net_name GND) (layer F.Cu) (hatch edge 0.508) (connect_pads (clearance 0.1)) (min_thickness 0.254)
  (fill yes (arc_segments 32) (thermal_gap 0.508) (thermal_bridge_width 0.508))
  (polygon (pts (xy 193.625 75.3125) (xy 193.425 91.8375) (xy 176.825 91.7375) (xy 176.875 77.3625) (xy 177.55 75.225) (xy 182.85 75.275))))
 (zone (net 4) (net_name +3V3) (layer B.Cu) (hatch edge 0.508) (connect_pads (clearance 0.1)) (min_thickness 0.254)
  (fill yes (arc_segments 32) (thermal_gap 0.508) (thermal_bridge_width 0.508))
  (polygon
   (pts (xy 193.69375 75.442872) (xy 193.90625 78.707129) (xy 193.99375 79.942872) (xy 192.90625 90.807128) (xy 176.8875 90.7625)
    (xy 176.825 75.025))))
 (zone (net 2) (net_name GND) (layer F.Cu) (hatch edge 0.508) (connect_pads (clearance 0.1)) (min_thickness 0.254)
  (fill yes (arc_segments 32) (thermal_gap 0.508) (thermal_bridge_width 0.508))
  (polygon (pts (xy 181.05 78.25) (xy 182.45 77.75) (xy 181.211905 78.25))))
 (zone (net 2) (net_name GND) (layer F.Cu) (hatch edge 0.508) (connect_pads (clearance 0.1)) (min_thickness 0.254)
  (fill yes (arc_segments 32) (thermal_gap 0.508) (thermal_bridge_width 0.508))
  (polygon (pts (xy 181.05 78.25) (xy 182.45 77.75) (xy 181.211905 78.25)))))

